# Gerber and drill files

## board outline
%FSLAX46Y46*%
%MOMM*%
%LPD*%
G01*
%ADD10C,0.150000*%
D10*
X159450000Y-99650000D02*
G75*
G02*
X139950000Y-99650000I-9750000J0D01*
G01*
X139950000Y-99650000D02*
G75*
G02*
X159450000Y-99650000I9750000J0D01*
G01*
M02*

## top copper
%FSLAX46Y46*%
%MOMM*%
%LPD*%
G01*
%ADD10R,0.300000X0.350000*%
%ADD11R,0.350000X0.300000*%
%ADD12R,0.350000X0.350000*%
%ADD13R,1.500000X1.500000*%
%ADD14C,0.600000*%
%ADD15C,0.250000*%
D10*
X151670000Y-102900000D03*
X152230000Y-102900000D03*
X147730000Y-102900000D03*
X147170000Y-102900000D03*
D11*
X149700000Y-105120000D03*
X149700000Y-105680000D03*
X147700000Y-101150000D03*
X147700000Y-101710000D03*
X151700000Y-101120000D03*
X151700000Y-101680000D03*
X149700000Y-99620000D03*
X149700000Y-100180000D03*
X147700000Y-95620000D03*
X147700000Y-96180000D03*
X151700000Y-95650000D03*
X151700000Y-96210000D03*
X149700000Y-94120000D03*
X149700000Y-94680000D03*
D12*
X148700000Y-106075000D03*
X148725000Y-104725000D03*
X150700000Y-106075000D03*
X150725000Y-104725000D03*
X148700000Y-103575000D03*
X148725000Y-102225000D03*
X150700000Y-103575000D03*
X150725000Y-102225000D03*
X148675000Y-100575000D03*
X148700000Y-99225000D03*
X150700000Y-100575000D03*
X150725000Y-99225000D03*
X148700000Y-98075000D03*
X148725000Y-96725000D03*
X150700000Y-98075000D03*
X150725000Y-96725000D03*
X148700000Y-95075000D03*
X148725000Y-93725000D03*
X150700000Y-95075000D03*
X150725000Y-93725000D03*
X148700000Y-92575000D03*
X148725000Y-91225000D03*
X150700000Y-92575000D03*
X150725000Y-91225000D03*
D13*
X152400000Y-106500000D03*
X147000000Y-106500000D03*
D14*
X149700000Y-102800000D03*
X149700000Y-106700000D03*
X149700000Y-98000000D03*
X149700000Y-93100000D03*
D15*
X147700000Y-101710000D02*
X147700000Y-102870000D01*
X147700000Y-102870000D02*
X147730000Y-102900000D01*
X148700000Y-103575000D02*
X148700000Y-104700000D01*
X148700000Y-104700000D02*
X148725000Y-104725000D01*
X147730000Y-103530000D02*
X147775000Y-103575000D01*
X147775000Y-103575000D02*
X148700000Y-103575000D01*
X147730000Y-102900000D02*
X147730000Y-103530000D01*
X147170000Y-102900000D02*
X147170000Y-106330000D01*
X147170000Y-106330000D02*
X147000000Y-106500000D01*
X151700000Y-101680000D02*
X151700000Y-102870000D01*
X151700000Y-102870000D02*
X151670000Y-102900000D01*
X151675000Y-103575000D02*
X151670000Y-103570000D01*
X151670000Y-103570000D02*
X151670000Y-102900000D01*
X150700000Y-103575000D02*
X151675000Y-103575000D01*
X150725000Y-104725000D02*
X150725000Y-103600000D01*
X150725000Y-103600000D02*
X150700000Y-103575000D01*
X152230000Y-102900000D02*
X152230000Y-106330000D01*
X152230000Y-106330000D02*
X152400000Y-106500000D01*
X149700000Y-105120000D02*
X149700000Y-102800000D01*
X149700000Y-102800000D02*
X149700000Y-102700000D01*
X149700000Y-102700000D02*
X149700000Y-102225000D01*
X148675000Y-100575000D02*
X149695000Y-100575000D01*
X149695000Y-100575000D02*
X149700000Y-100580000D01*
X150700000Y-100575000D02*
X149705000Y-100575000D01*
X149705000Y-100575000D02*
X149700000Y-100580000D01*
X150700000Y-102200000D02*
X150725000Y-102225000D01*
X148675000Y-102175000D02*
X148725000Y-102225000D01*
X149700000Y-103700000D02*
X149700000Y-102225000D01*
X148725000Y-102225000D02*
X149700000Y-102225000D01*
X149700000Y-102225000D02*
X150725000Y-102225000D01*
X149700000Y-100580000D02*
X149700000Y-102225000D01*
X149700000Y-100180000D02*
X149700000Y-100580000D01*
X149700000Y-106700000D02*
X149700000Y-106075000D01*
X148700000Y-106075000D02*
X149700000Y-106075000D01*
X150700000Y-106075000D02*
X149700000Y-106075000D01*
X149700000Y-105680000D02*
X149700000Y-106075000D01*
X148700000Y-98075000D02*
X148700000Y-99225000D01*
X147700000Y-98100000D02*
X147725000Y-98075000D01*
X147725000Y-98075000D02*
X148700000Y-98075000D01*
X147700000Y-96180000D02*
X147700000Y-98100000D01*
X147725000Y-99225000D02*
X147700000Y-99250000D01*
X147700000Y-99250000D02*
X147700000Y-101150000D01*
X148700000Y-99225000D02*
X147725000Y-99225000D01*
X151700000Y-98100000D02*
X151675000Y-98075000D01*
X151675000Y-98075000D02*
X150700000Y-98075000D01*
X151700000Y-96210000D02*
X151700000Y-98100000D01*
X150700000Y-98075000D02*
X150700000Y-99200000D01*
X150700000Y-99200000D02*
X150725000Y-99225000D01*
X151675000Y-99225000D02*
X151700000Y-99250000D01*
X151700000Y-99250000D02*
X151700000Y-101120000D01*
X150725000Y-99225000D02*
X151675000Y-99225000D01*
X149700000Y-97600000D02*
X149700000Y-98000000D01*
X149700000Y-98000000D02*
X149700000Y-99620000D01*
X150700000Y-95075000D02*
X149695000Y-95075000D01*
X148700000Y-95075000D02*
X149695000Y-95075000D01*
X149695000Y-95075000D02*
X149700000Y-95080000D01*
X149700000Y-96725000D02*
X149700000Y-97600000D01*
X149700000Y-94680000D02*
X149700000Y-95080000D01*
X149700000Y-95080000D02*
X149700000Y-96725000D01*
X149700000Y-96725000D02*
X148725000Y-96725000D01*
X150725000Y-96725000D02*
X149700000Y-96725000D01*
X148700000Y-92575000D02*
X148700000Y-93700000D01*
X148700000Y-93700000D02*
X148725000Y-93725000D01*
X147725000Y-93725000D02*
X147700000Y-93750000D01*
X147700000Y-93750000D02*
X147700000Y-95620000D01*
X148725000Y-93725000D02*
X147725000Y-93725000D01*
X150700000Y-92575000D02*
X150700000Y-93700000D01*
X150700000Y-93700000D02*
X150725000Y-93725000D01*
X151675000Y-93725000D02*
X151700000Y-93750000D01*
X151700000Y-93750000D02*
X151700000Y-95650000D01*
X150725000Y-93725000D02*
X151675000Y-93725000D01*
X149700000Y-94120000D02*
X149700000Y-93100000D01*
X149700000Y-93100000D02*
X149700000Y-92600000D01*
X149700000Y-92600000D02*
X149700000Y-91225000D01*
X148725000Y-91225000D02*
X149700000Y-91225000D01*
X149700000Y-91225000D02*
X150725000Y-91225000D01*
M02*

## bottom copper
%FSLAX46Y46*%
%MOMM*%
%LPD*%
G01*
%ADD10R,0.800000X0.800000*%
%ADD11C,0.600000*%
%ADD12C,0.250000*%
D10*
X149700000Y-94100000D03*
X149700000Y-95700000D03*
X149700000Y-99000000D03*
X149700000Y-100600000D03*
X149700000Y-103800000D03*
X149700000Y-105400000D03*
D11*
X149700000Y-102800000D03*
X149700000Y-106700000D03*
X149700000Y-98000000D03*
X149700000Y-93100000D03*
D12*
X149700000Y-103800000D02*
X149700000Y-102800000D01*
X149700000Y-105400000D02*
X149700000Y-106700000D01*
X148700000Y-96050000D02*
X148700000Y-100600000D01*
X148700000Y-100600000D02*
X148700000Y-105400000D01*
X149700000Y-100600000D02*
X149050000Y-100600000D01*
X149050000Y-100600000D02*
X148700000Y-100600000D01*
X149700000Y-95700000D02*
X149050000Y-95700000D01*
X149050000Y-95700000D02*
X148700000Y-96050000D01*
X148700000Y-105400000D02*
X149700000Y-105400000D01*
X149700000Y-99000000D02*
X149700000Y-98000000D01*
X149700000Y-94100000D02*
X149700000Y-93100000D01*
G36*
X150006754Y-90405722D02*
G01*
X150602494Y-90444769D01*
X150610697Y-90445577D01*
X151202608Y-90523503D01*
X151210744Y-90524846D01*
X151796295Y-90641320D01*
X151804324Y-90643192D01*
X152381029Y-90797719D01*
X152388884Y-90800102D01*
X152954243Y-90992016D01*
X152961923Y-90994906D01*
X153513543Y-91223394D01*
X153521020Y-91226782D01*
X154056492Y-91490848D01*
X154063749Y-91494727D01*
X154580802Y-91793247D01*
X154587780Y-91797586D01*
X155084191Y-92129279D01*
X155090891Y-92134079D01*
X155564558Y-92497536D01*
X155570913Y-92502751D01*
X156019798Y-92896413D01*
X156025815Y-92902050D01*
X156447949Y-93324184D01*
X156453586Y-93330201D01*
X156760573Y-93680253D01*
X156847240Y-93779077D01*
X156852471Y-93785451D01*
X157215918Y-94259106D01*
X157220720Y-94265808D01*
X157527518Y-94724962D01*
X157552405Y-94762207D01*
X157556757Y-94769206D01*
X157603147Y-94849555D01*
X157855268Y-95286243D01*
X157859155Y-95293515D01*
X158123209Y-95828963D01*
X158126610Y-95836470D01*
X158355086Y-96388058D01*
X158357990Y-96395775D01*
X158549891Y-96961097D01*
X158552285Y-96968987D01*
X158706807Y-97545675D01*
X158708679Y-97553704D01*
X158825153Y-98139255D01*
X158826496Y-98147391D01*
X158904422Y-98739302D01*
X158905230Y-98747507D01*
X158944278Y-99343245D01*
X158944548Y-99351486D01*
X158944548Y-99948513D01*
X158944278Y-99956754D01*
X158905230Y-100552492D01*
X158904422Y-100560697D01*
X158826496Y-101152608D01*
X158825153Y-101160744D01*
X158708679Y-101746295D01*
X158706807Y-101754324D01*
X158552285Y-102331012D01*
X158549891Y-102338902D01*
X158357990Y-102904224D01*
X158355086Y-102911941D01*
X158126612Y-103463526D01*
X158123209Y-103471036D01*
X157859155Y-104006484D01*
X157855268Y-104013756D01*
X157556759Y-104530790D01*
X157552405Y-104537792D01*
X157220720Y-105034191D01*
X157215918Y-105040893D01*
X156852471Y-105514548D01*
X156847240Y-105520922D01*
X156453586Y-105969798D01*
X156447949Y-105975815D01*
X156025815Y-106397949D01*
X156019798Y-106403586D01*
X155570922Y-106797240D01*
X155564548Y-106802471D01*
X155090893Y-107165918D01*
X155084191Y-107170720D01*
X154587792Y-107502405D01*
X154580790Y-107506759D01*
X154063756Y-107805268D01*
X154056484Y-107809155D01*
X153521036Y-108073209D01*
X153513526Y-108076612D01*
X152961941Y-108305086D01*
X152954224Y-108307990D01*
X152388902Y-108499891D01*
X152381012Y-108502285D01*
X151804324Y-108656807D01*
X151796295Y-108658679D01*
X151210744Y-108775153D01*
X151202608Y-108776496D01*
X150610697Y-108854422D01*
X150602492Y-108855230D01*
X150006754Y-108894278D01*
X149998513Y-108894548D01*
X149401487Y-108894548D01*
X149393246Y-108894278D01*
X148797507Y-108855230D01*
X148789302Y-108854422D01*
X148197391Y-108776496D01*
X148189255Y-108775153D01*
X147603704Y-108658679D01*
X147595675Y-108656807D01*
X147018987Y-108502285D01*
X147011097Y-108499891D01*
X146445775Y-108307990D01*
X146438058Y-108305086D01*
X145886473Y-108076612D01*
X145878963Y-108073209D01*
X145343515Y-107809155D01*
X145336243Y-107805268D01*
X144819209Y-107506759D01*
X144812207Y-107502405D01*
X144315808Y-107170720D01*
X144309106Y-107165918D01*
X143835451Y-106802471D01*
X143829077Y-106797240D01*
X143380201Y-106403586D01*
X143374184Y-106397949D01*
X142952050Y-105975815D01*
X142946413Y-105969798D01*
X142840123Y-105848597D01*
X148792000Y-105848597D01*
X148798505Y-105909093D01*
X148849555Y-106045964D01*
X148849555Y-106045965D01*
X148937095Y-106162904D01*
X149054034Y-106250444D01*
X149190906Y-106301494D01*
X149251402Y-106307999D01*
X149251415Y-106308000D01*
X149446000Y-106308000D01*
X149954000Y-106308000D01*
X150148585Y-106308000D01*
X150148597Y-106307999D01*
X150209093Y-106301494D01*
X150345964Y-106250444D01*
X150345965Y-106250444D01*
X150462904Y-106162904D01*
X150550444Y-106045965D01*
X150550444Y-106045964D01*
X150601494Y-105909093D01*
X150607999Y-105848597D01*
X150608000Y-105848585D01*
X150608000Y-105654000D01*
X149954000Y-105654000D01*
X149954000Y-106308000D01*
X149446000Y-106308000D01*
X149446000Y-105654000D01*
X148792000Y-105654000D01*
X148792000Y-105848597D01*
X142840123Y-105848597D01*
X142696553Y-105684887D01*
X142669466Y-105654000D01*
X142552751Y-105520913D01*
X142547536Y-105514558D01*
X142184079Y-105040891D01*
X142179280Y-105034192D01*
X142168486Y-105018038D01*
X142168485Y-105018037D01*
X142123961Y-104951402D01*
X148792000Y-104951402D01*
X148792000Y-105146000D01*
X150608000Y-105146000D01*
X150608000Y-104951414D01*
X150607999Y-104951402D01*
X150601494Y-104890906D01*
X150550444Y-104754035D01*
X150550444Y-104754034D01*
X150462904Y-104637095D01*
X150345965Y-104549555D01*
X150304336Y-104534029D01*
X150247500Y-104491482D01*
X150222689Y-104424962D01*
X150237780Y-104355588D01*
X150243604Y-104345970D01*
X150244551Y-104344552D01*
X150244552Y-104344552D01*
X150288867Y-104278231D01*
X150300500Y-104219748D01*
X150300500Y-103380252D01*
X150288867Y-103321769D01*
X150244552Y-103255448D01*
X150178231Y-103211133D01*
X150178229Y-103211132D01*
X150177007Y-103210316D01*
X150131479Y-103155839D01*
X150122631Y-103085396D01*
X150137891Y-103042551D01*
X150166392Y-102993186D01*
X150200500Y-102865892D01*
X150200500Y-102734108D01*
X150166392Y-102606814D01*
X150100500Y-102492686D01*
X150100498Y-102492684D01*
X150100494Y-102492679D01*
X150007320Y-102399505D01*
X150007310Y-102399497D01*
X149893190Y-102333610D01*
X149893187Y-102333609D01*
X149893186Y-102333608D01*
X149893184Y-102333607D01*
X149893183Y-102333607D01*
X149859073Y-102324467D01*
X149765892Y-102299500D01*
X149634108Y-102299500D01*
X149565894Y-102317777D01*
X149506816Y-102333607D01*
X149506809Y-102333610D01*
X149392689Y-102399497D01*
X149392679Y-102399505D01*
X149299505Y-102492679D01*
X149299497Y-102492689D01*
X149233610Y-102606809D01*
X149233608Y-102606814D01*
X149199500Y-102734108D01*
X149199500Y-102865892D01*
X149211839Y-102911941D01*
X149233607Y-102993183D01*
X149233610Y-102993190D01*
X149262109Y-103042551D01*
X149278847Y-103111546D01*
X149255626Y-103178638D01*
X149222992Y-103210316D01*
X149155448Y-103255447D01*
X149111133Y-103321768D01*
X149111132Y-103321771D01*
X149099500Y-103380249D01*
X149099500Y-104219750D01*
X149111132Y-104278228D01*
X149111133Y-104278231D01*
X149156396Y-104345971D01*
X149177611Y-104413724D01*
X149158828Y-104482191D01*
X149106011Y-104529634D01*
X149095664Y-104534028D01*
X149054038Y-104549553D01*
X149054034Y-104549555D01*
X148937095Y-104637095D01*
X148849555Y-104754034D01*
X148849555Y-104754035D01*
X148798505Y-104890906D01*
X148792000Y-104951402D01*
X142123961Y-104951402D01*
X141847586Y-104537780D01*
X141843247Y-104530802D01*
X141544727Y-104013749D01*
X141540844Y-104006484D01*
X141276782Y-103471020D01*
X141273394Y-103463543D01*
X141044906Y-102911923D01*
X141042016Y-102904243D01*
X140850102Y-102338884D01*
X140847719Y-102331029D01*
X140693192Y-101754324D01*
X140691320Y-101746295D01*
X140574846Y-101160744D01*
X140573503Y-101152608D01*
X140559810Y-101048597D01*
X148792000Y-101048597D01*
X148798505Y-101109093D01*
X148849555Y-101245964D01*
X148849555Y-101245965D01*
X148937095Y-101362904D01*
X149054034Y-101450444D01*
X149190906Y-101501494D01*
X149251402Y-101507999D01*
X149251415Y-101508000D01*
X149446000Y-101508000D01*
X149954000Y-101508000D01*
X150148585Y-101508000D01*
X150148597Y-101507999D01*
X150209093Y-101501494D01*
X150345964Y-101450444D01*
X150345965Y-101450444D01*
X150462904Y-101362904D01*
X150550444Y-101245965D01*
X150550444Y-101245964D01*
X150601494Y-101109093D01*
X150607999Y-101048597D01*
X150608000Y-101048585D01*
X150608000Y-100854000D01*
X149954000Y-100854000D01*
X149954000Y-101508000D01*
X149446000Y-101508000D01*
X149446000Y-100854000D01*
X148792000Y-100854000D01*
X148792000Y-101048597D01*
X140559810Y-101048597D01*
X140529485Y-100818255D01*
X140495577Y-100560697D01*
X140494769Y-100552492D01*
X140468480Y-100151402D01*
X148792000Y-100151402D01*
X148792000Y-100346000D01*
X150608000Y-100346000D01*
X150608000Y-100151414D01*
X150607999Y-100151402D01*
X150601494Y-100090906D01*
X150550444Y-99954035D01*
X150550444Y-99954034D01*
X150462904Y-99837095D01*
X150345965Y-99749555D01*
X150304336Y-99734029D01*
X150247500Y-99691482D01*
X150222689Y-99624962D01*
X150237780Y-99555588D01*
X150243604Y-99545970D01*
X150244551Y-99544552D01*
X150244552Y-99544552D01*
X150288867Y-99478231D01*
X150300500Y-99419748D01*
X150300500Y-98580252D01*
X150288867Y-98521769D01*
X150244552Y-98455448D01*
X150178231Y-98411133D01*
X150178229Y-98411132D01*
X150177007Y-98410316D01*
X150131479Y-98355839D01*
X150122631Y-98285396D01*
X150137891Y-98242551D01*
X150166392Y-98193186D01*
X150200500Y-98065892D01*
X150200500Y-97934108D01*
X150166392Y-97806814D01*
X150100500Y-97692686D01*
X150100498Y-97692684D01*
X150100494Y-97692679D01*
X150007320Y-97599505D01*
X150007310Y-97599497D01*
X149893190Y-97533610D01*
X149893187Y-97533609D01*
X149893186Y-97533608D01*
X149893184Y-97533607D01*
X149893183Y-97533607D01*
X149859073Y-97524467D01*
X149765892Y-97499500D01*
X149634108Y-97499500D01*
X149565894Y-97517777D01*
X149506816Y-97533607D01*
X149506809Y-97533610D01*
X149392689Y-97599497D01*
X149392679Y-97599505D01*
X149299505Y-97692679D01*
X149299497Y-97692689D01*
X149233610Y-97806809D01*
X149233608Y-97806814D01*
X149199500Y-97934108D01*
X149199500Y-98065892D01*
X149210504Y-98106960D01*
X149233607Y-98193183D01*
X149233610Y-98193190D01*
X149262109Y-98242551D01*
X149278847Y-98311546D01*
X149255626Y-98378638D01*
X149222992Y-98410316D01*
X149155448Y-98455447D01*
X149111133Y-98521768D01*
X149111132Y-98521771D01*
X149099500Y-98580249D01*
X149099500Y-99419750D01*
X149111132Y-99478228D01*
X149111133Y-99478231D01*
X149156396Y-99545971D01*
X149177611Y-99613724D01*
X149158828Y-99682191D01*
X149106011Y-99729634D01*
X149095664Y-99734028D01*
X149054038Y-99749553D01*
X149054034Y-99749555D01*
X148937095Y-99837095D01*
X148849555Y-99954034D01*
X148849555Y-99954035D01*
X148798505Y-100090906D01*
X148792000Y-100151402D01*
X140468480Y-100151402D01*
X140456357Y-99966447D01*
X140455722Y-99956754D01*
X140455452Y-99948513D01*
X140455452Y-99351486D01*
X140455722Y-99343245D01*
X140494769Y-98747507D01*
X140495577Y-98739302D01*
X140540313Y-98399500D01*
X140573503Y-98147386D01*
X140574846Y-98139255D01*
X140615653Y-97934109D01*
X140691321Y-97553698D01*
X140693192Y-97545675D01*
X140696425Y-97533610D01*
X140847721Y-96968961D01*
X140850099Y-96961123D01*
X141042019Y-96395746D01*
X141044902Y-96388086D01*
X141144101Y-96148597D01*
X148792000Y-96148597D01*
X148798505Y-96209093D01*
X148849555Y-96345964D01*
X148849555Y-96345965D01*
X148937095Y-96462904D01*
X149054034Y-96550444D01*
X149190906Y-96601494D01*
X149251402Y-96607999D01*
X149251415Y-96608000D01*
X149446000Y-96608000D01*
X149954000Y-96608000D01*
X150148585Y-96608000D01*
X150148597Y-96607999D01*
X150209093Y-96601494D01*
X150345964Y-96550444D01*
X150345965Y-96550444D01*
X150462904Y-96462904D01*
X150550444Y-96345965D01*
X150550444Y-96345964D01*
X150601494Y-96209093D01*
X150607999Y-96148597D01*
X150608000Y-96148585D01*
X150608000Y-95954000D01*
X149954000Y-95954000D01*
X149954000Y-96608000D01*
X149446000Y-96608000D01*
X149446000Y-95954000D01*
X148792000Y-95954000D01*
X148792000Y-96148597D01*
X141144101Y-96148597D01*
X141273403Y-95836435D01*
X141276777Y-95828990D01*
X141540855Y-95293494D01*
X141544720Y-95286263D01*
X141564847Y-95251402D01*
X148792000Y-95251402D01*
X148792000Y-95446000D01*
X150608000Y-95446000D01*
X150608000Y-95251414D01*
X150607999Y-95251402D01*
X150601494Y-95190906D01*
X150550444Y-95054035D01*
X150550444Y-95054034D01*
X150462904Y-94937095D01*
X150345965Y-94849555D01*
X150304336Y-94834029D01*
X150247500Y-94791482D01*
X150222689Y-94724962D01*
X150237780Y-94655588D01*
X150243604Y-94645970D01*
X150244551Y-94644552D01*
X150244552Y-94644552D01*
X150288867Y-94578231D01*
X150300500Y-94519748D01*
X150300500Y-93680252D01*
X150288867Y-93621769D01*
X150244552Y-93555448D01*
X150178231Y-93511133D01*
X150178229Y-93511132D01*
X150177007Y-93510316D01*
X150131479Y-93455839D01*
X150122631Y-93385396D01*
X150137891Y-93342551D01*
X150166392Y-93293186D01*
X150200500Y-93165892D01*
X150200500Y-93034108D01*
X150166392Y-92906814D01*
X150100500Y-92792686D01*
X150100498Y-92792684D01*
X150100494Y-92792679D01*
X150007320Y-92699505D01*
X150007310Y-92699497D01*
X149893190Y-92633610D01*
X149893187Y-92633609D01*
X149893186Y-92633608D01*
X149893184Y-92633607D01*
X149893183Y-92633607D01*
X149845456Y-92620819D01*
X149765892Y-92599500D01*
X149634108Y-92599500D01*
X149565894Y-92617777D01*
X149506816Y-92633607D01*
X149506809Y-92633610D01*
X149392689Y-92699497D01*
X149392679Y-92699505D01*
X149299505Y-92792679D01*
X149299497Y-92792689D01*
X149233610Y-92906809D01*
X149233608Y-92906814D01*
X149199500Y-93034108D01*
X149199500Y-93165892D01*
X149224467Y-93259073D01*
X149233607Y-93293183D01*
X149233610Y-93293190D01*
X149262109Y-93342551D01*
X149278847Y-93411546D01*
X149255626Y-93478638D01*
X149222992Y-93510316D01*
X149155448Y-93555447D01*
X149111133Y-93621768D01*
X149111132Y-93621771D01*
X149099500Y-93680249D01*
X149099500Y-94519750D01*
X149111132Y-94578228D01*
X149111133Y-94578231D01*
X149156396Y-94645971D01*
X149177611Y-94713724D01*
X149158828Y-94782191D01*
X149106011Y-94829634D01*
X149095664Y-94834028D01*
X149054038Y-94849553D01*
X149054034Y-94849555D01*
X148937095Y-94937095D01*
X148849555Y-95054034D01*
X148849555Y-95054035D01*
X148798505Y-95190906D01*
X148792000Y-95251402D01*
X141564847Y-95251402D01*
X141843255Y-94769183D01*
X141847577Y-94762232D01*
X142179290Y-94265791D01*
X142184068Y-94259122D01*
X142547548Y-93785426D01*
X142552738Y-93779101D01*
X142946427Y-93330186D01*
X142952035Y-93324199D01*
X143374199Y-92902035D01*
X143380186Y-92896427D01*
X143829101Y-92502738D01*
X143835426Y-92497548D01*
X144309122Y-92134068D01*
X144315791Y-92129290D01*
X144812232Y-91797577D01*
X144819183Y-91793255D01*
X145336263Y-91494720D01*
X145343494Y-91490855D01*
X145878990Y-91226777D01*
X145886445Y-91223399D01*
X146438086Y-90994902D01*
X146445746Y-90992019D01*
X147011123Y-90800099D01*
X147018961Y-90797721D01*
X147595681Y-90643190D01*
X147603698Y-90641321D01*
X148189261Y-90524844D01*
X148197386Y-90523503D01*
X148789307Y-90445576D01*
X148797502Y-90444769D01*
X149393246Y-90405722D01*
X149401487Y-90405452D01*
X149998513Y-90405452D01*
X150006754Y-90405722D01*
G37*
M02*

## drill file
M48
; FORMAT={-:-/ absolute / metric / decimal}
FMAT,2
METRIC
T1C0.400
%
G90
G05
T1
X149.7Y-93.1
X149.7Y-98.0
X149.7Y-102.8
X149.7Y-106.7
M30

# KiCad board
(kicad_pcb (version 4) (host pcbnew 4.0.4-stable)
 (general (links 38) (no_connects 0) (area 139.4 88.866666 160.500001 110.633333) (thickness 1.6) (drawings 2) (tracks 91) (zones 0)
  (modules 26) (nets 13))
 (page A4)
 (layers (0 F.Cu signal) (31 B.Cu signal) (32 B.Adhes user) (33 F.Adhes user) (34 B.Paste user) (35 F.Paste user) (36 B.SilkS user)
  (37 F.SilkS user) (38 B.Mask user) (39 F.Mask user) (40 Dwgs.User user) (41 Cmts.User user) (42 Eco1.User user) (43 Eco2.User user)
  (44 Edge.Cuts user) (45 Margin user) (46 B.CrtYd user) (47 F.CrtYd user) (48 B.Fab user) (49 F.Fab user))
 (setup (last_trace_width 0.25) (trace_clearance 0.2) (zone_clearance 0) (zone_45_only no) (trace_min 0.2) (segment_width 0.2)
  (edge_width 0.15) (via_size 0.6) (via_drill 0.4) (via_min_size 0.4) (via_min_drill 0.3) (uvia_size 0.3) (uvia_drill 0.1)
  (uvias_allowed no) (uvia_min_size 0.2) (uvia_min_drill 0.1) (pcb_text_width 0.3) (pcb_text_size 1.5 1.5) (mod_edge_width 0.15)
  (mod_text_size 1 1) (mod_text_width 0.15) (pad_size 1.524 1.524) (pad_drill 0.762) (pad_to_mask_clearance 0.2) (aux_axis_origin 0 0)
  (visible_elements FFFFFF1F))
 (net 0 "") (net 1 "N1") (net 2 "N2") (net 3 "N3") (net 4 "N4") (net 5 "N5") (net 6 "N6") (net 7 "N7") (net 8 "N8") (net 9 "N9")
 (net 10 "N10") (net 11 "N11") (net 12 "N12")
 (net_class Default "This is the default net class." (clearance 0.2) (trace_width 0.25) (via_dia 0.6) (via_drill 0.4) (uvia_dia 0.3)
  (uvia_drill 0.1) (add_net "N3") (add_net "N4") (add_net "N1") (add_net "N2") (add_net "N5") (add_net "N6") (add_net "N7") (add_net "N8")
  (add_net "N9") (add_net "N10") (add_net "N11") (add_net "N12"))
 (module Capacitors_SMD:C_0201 (layer F.Cu) (at 151.95 102.9)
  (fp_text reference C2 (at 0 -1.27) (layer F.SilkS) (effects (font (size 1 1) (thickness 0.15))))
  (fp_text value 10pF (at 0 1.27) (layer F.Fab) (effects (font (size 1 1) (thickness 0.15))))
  (pad 1 smd rect (at -0.28 0) (size 0.3 0.35) (layers F.Cu F.Paste F.Mask) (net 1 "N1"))
  (pad 2 smd rect (at 0.28 0) (size 0.3 0.35) (layers F.Cu F.Paste F.Mask) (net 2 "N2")))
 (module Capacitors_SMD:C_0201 (layer F.Cu) (at 147.45 102.9 180)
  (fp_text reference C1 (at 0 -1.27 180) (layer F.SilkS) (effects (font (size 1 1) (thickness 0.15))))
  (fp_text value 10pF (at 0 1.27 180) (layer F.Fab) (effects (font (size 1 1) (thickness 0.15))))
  (pad 1 smd rect (at -0.28 0 180) (size 0.3 0.35) (layers F.Cu F.Paste F.Mask) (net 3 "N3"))
  (pad 2 smd rect (at 0.28 0 180) (size 0.3 0.35) (layers F.Cu F.Paste F.Mask) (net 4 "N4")))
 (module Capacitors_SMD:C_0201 (layer F.Cu) (at 149.7 105.4 270)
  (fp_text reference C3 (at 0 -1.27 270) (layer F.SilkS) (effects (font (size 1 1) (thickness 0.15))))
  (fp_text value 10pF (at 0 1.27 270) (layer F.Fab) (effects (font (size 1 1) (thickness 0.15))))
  (pad 1 smd rect (at -0.28 0 270) (size 0.3 0.35) (layers F.Cu F.Paste F.Mask) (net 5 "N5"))
  (pad 2 smd rect (at 0.28 0 270) (size 0.3 0.35) (layers F.Cu F.Paste F.Mask) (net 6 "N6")))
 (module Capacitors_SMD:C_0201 (layer F.Cu) (at 147.7 101.43 270)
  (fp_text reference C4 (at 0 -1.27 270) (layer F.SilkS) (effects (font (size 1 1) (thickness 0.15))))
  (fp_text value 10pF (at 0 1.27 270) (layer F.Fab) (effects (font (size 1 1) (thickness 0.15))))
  (pad 1 smd rect (at -0.28 0 270) (size 0.3 0.35) (layers F.Cu F.Paste F.Mask) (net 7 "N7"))
  (pad 2 smd rect (at 0.28 0 270) (size 0.3 0.35) (layers F.Cu F.Paste F.Mask) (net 3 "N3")))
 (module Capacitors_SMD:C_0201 (layer F.Cu) (at 151.7 101.4 270)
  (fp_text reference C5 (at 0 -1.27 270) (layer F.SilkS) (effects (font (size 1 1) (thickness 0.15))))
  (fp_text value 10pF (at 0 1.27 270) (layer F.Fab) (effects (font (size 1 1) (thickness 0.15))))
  (pad 1 smd rect (at -0.28 0 270) (size 0.3 0.35) (layers F.Cu F.Paste F.Mask) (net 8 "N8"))
  (pad 2 smd rect (at 0.28 0 270) (size 0.3 0.35) (layers F.Cu F.Paste F.Mask) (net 1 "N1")))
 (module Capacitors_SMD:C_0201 (layer F.Cu) (at 149.7 99.9 270)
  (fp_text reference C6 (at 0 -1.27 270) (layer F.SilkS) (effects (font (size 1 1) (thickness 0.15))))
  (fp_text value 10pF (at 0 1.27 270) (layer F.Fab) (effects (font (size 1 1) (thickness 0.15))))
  (pad 1 smd rect (at -0.28 0 270) (size 0.3 0.35) (layers F.Cu F.Paste F.Mask) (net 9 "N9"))
  (pad 2 smd rect (at 0.28 0 270) (size 0.3 0.35) (layers F.Cu F.Paste F.Mask) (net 5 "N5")))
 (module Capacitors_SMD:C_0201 (layer F.Cu) (at 147.7 95.9 270)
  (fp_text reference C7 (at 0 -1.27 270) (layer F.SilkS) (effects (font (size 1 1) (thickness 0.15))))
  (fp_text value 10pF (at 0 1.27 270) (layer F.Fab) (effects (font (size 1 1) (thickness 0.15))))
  (pad 1 smd rect (at -0.28 0 270) (size 0.3 0.35) (layers F.Cu F.Paste F.Mask) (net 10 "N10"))
  (pad 2 smd rect (at 0.28 0 270) (size 0.3 0.35) (layers F.Cu F.Paste F.Mask) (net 7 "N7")))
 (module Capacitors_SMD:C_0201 (layer F.Cu) (at 151.7 95.93 270)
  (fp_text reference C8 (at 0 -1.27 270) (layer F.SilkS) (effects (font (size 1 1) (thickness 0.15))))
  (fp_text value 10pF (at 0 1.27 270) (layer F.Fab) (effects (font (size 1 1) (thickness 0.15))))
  (pad 1 smd rect (at -0.28 0 270) (size 0.3 0.35) (layers F.Cu F.Paste F.Mask) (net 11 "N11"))
  (pad 2 smd rect (at 0.28 0 270) (size 0.3 0.35) (layers F.Cu F.Paste F.Mask) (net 8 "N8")))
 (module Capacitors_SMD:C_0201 (layer F.Cu) (at 149.7 94.4 270)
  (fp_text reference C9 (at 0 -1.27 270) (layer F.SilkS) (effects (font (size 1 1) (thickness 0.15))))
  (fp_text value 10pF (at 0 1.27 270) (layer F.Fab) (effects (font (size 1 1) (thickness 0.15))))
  (pad 1 smd rect (at -0.28 0 270) (size 0.3 0.35) (layers F.Cu F.Paste F.Mask) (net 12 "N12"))
  (pad 2 smd rect (at 0.28 0 270) (size 0.3 0.35) (layers F.Cu F.Paste F.Mask) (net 9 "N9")))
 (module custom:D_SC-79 (layer F.Cu) (at 148.7 105.4 270)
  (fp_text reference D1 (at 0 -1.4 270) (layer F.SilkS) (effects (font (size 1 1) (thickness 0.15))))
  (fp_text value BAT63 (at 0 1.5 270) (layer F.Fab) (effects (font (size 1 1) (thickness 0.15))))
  (pad 2 smd rect (at 0.675 0 270) (size 0.35 0.35) (layers F.Cu F.Paste F.Mask) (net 6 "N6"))
  (pad 1 smd rect (at -0.675 -0.025 270) (size 0.35 0.35) (layers F.Cu F.Paste F.Mask) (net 3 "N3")))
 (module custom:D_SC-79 (layer F.Cu) (at 150.7 105.4 270)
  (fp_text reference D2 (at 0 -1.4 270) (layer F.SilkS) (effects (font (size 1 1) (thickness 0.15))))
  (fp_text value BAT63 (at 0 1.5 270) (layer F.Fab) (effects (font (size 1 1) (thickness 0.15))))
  (pad 2 smd rect (at 0.675 0 270) (size 0.35 0.35) (layers F.Cu F.Paste F.Mask) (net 6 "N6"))
  (pad 1 smd rect (at -0.675 -0.025 270) (size 0.35 0.35) (layers F.Cu F.Paste F.Mask) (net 1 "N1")))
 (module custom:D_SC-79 (layer F.Cu) (at 148.7 102.9 270)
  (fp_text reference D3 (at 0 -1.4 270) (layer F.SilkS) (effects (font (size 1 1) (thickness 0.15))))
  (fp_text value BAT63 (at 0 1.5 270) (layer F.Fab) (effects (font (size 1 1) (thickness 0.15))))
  (pad 2 smd rect (at 0.675 0 270) (size 0.35 0.35) (layers F.Cu F.Paste F.Mask) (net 3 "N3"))
  (pad 1 smd rect (at -0.675 -0.025 270) (size 0.35 0.35) (layers F.Cu F.Paste F.Mask) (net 5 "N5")))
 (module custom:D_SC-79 (layer F.Cu) (at 150.7 102.9 270)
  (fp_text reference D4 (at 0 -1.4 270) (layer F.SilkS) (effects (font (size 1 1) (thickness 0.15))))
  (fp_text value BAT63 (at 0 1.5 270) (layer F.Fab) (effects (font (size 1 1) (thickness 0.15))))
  (pad 2 smd rect (at 0.675 0 270) (size 0.35 0.35) (layers F.Cu F.Paste F.Mask) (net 1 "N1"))
  (pad 1 smd rect (at -0.675 -0.025 270) (size 0.35 0.35) (layers F.Cu F.Paste F.Mask) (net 5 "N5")))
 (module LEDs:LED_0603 (layer B.Cu) (at 149.7 94.9 90)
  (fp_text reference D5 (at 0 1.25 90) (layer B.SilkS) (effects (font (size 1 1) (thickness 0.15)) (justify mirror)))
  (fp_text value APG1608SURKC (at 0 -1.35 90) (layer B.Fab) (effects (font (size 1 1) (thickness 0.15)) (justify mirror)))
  (pad 2 smd rect (at 0.8 0 270) (size 0.8 0.8) (layers B.Cu B.Paste B.Mask) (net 12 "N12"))
  (pad 1 smd rect (at -0.8 0 270) (size 0.8 0.8) (layers B.Cu B.Paste B.Mask) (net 6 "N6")))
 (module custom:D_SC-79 (layer F.Cu) (at 148.675 99.9 270)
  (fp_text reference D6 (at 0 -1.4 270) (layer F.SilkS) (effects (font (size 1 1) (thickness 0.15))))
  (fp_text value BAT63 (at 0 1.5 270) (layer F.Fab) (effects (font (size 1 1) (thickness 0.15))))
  (pad 2 smd rect (at 0.675 0 270) (size 0.35 0.35) (layers F.Cu F.Paste F.Mask) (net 5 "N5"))
  (pad 1 smd rect (at -0.675 -0.025 270) (size 0.35 0.35) (layers F.Cu F.Paste F.Mask) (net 7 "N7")))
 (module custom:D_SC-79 (layer F.Cu) (at 150.7 99.9 270)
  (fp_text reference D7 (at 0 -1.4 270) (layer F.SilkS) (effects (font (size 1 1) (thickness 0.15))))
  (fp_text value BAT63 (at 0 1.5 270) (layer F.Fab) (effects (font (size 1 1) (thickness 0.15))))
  (pad 2 smd rect (at 0.675 0 270) (size 0.35 0.35) (layers F.Cu F.Paste F.Mask) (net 5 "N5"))
  (pad 1 smd rect (at -0.675 -0.025 270) (size 0.35 0.35) (layers F.Cu F.Paste F.Mask) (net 8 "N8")))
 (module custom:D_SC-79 (layer F.Cu) (at 148.7 97.4 270)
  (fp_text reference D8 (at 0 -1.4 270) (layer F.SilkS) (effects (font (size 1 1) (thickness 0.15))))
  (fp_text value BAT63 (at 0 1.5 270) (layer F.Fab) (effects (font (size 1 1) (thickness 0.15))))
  (pad 2 smd rect (at 0.675 0 270) (size 0.35 0.35) (layers F.Cu F.Paste F.Mask) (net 7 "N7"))
  (pad 1 smd rect (at -0.675 -0.025 270) (size 0.35 0.35) (layers F.Cu F.Paste F.Mask) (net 9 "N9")))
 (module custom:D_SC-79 (layer F.Cu) (at 150.7 97.4 270)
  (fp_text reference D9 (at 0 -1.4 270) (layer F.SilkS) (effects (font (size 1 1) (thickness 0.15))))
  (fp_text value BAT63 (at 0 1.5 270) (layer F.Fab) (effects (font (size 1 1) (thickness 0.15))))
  (pad 2 smd rect (at 0.675 0 270) (size 0.35 0.35) (layers F.Cu F.Paste F.Mask) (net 8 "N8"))
  (pad 1 smd rect (at -0.675 -0.025 270) (size 0.35 0.35) (layers F.Cu F.Paste F.Mask) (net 9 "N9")))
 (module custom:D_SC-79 (layer F.Cu) (at 148.7 94.4 270)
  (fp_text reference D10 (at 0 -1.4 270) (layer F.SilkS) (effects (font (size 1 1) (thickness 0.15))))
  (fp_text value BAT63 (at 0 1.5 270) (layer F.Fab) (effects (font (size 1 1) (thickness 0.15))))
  (pad 2 smd rect (at 0.675 0 270) (size 0.35 0.35) (layers F.Cu F.Paste F.Mask) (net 9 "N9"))
  (pad 1 smd rect (at -0.675 -0.025 270) (size 0.35 0.35) (layers F.Cu F.Paste F.Mask) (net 10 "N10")))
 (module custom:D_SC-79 (layer F.Cu) (at 150.7 94.4 270)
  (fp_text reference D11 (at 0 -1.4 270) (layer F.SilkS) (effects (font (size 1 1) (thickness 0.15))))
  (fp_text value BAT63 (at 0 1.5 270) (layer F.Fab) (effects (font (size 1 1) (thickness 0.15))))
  (pad 2 smd rect (at 0.675 0 270) (size 0.35 0.35) (layers F.Cu F.Paste F.Mask) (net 9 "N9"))
  (pad 1 smd rect (at -0.675 -0.025 270) (size 0.35 0.35) (layers F.Cu F.Paste F.Mask) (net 11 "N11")))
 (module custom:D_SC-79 (layer F.Cu) (at 148.7 91.9 270)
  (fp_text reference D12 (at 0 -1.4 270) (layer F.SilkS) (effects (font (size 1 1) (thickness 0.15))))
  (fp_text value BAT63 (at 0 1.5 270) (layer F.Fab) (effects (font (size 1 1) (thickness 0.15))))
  (pad 2 smd rect (at 0.675 0 270) (size 0.35 0.35) (layers F.Cu F.Paste F.Mask) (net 10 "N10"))
  (pad 1 smd rect (at -0.675 -0.025 270) (size 0.35 0.35) (layers F.Cu F.Paste F.Mask) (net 12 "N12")))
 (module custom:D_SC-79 (layer F.Cu) (at 150.7 91.9 270)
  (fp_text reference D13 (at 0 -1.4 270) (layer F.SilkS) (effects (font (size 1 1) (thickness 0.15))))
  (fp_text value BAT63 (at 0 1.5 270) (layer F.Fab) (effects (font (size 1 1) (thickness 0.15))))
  (pad 2 smd rect (at 0.675 0 270) (size 0.35 0.35) (layers F.Cu F.Paste F.Mask) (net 11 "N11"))
  (pad 1 smd rect (at -0.675 -0.025 270) (size 0.35 0.35) (layers F.Cu F.Paste F.Mask) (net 12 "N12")))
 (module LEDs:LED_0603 (layer B.Cu) (at 149.7 99.8 90)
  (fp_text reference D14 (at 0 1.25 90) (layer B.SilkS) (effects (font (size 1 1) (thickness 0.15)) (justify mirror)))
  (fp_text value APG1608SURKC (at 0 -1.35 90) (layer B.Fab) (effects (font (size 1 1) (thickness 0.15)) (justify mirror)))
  (pad 2 smd rect (at 0.8 0 270) (size 0.8 0.8) (layers B.Cu B.Paste B.Mask) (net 9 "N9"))
  (pad 1 smd rect (at -0.8 0 270) (size 0.8 0.8) (layers B.Cu B.Paste B.Mask) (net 6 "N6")))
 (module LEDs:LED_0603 (layer B.Cu) (at 149.7 104.6 90)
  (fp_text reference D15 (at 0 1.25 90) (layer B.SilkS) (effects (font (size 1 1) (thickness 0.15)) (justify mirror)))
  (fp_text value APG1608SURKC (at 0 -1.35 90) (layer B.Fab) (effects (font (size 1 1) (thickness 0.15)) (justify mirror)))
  (pad 2 smd rect (at 0.8 0 270) (size 0.8 0.8) (layers B.Cu B.Paste B.Mask) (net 5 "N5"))
  (pad 1 smd rect (at -0.8 0 270) (size 0.8 0.8) (layers B.Cu B.Paste B.Mask) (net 6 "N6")))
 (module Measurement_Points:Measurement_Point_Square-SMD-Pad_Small (layer F.Cu) (at 152.4 106.5)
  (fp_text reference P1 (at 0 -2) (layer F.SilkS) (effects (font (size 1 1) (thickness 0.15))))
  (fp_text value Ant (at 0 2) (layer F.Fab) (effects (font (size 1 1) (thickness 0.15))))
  (pad 1 smd rect (at 0 0) (size 1.5 1.5) (layers F.Cu F.Mask) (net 2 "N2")))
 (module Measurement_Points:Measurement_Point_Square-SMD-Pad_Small (layer F.Cu) (at 147 106.5)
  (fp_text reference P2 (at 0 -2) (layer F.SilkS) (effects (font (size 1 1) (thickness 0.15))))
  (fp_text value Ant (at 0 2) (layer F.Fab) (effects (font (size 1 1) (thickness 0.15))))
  (pad 1 smd rect (at 0 0) (size 1.5 1.5) (layers F.Cu F.Mask) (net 4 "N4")))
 (gr_circle (center 149.7 99.65) (end 149.7 109.4) (layer Edge.Cuts) (width 0.15))
 (segment (start 147.7 101.71) (end 147.7 102.87) (width 0.25) (layer F.Cu) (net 3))
 (segment (start 147.7 102.87) (end 147.73 102.9) (width 0.25) (layer F.Cu) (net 3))
 (segment (start 148.7 103.575) (end 148.7 104.7) (width 0.25) (layer F.Cu) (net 3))
 (segment (start 148.7 104.7) (end 148.725 104.725) (width 0.25) (layer F.Cu) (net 3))
 (segment (start 147.73 103.53) (end 147.775 103.575) (width 0.25) (layer F.Cu) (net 3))
 (segment (start 147.775 103.575) (end 148.7 103.575) (width 0.25) (layer F.Cu) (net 3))
 (segment (start 147.73 102.9) (end 147.73 103.53) (width 0.25) (layer F.Cu) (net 3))
 (segment (start 147.17 102.9) (end 147.17 106.33) (width 0.25) (layer F.Cu) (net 4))
 (segment (start 147.17 106.33) (end 147 106.5) (width 0.25) (layer F.Cu) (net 4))
 (segment (start 151.7 101.68) (end 151.7 102.87) (width 0.25) (layer F.Cu) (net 1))
 (segment (start 151.7 102.87) (end 151.67 102.9) (width 0.25) (layer F.Cu) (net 1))
 (segment (start 151.675 103.575) (end 151.67 103.57) (width 0.25) (layer F.Cu) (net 1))
 (segment (start 151.67 103.57) (end 151.67 102.9) (width 0.25) (layer F.Cu) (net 1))
 (segment (start 150.7 103.575) (end 151.675 103.575) (width 0.25) (layer F.Cu) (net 1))
 (segment (start 150.725 104.725) (end 150.725 103.6) (width 0.25) (layer F.Cu) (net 1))
 (segment (start 150.725 103.6) (end 150.7 103.575) (width 0.25) (layer F.Cu) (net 1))
 (segment (start 152.23 102.9) (end 152.23 106.33) (width 0.25) (layer F.Cu) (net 2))
 (segment (start 152.23 106.33) (end 152.4 106.5) (width 0.25) (layer F.Cu) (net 2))
 (segment (start 149.7 105.12) (end 149.7 102.8) (width 0.25) (layer F.Cu) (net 5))
 (segment (start 149.7 102.8) (end 149.7 102.7) (width 0.25) (layer F.Cu) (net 5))
 (segment (start 149.7 103.8) (end 149.7 102.8) (width 0.25) (layer B.Cu) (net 5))
 (via (at 149.7 102.8) (size 0.6) (drill 0.4) (layers F.Cu B.Cu) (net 5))
 (segment (start 149.7 102.7) (end 149.7 102.225) (width 0.25) (layer F.Cu) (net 5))
 (segment (start 148.675 100.575) (end 149.695 100.575) (width 0.25) (layer F.Cu) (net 5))
 (segment (start 149.695 100.575) (end 149.7 100.58) (width 0.25) (layer F.Cu) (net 5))
 (segment (start 150.7 100.575) (end 149.705 100.575) (width 0.25) (layer F.Cu) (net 5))
 (segment (start 149.705 100.575) (end 149.7 100.58) (width 0.25) (layer F.Cu) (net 5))
 (segment (start 150.7 102.2) (end 150.725 102.225) (width 0.25) (layer F.Cu) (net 5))
 (segment (start 148.675 102.175) (end 148.725 102.225) (width 0.25) (layer F.Cu) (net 5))
 (segment (start 149.7 103.7) (end 149.7 102.225) (width 0.25) (layer F.Cu) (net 5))
 (segment (start 148.725 102.225) (end 149.7 102.225) (width 0.25) (layer F.Cu) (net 5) (status 10))
 (segment (start 149.7 102.225) (end 150.725 102.225) (width 0.25) (layer F.Cu) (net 5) (status 20))
 (segment (start 149.7 100.58) (end 149.7 102.225) (width 0.25) (layer F.Cu) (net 5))
 (segment (start 149.7 100.18) (end 149.7 100.58) (width 0.25) (layer F.Cu) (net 5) (status 10))
 (segment (start 149.7 106.7) (end 149.7 106.075) (width 0.25) (layer F.Cu) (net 6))
 (segment (start 149.7 105.4) (end 149.7 106.7) (width 0.25) (layer B.Cu) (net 6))
 (via (at 149.7 106.7) (size 0.6) (drill 0.4) (layers F.Cu B.Cu) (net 6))
 (segment (start 148.7 96.05) (end 148.7 100.6) (width 0.25) (layer B.Cu) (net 6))
 (segment (start 148.7 100.6) (end 148.7 105.4) (width 0.25) (layer B.Cu) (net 6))
 (segment (start 149.7 100.6) (end 149.05 100.6) (width 0.25) (layer B.Cu) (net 6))
 (segment (start 149.05 100.6) (end 148.7 100.6) (width 0.25) (layer B.Cu) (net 6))
 (segment (start 149.7 95.7) (end 149.05 95.7) (width 0.25) (layer B.Cu) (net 6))
 (segment (start 149.05 95.7) (end 148.7 96.05) (width 0.25) (layer B.Cu) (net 6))
 (segment (start 148.7 105.4) (end 149.7 105.4) (width 0.25) (layer B.Cu) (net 6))
 (segment (start 148.7 106.075) (end 149.7 106.075) (width 0.25) (layer F.Cu) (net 6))
 (segment (start 150.7 106.075) (end 149.7 106.075) (width 0.25) (layer F.Cu) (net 6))
 (segment (start 149.7 105.68) (end 149.7 106.075) (width 0.25) (layer F.Cu) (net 6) (status 10))
 (segment (start 148.7 98.075) (end 148.7 99.225) (width 0.25) (layer F.Cu) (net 7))
 (segment (start 147.7 98.1) (end 147.725 98.075) (width 0.25) (layer F.Cu) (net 7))
 (segment (start 147.725 98.075) (end 148.7 98.075) (width 0.25) (layer F.Cu) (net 7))
 (segment (start 147.7 96.18) (end 147.7 98.1) (width 0.25) (layer F.Cu) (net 7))
 (segment (start 147.725 99.225) (end 147.7 99.25) (width 0.25) (layer F.Cu) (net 7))
 (segment (start 147.7 99.25) (end 147.7 101.15) (width 0.25) (layer F.Cu) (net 7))
 (segment (start 148.7 99.225) (end 147.725 99.225) (width 0.25) (layer F.Cu) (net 7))
 (segment (start 151.7 98.1) (end 151.675 98.075) (width 0.25) (layer F.Cu) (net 8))
 (segment (start 151.675 98.075) (end 150.7 98.075) (width 0.25) (layer F.Cu) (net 8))
 (segment (start 151.7 96.21) (end 151.7 98.1) (width 0.25) (layer F.Cu) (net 8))
 (segment (start 150.7 98.075) (end 150.7 99.2) (width 0.25) (layer F.Cu) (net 8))
 (segment (start 150.7 99.2) (end 150.725 99.225) (width 0.25) (layer F.Cu) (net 8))
 (segment (start 151.675 99.225) (end 151.7 99.25) (width 0.25) (layer F.Cu) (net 8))
 (segment (start 151.7 99.25) (end 151.7 101.12) (width 0.25) (layer F.Cu) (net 8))
 (segment (start 150.725 99.225) (end 151.675 99.225) (width 0.25) (layer F.Cu) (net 8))
 (segment (start 149.7 97.6) (end 149.7 98) (width 0.25) (layer F.Cu) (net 9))
 (segment (start 149.7 98) (end 149.7 99.62) (width 0.25) (layer F.Cu) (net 9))
 (segment (start 149.7 99) (end 149.7 98) (width 0.25) (layer B.Cu) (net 9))
 (via (at 149.7 98) (size 0.6) (drill 0.4) (layers F.Cu B.Cu) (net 9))
 (segment (start 150.7 95.075) (end 149.695 95.075) (width 0.25) (layer F.Cu) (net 9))
 (segment (start 148.7 95.075) (end 149.695 95.075) (width 0.25) (layer F.Cu) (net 9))
 (segment (start 149.695 95.075) (end 149.7 95.08) (width 0.25) (layer F.Cu) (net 9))
 (segment (start 149.7 96.725) (end 149.7 97.6) (width 0.25) (layer F.Cu) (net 9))
 (segment (start 149.7 94.68) (end 149.7 95.08) (width 0.25) (layer F.Cu) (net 9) (status 10))
 (segment (start 149.7 95.08) (end 149.7 96.725) (width 0.25) (layer F.Cu) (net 9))
 (segment (start 149.7 96.725) (end 148.725 96.725) (width 0.25) (layer F.Cu) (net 9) (status 20))
 (segment (start 150.725 96.725) (end 149.7 96.725) (width 0.25) (layer F.Cu) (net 9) (status 10))
 (segment (start 148.7 92.575) (end 148.7 93.7) (width 0.25) (layer F.Cu) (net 10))
 (segment (start 148.7 93.7) (end 148.725 93.725) (width 0.25) (layer F.Cu) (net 10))
 (segment (start 147.725 93.725) (end 147.7 93.75) (width 0.25) (layer F.Cu) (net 10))
 (segment (start 147.7 93.75) (end 147.7 95.62) (width 0.25) (layer F.Cu) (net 10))
 (segment (start 148.725 93.725) (end 147.725 93.725) (width 0.25) (layer F.Cu) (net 10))
 (segment (start 150.7 92.575) (end 150.7 93.7) (width 0.25) (layer F.Cu) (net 11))
 (segment (start 150.7 93.7) (end 150.725 93.725) (width 0.25) (layer F.Cu) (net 11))
 (segment (start 151.675 93.725) (end 151.7 93.75) (width 0.25) (layer F.Cu) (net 11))
 (segment (start 151.7 93.75) (end 151.7 95.65) (width 0.25) (layer F.Cu) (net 11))
 (segment (start 150.725 93.725) (end 151.675 93.725) (width 0.25) (layer F.Cu) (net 11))
 (segment (start 149.7 94.12) (end 149.7 93.1) (width 0.25) (layer F.Cu) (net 12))
 (segment (start 149.7 93.1) (end 149.7 92.6) (width 0.25) (layer F.Cu) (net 12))
 (segment (start 149.7 94.1) (end 149.7 93.1) (width 0.25) (layer B.Cu) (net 12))
 (via (at 149.7 93.1) (size 0.6) (drill 0.4) (layers F.Cu B.Cu) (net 12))
 (segment (start 149.7 92.6) (end 149.7 91.225) (width 0.25) (layer F.Cu) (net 12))
 (segment (start 148.725 91.225) (end 149.7 91.225) (width 0.25) (layer F.Cu) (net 12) (status 10))
 (segment (start 149.7 91.225) (end 150.725 91.225) (width 0.25) (layer F.Cu) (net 12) (status 20))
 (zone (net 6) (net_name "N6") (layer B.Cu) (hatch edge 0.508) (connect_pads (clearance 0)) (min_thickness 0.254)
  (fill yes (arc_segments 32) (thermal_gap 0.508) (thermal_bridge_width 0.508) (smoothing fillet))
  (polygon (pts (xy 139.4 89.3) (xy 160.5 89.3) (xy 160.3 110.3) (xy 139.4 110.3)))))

